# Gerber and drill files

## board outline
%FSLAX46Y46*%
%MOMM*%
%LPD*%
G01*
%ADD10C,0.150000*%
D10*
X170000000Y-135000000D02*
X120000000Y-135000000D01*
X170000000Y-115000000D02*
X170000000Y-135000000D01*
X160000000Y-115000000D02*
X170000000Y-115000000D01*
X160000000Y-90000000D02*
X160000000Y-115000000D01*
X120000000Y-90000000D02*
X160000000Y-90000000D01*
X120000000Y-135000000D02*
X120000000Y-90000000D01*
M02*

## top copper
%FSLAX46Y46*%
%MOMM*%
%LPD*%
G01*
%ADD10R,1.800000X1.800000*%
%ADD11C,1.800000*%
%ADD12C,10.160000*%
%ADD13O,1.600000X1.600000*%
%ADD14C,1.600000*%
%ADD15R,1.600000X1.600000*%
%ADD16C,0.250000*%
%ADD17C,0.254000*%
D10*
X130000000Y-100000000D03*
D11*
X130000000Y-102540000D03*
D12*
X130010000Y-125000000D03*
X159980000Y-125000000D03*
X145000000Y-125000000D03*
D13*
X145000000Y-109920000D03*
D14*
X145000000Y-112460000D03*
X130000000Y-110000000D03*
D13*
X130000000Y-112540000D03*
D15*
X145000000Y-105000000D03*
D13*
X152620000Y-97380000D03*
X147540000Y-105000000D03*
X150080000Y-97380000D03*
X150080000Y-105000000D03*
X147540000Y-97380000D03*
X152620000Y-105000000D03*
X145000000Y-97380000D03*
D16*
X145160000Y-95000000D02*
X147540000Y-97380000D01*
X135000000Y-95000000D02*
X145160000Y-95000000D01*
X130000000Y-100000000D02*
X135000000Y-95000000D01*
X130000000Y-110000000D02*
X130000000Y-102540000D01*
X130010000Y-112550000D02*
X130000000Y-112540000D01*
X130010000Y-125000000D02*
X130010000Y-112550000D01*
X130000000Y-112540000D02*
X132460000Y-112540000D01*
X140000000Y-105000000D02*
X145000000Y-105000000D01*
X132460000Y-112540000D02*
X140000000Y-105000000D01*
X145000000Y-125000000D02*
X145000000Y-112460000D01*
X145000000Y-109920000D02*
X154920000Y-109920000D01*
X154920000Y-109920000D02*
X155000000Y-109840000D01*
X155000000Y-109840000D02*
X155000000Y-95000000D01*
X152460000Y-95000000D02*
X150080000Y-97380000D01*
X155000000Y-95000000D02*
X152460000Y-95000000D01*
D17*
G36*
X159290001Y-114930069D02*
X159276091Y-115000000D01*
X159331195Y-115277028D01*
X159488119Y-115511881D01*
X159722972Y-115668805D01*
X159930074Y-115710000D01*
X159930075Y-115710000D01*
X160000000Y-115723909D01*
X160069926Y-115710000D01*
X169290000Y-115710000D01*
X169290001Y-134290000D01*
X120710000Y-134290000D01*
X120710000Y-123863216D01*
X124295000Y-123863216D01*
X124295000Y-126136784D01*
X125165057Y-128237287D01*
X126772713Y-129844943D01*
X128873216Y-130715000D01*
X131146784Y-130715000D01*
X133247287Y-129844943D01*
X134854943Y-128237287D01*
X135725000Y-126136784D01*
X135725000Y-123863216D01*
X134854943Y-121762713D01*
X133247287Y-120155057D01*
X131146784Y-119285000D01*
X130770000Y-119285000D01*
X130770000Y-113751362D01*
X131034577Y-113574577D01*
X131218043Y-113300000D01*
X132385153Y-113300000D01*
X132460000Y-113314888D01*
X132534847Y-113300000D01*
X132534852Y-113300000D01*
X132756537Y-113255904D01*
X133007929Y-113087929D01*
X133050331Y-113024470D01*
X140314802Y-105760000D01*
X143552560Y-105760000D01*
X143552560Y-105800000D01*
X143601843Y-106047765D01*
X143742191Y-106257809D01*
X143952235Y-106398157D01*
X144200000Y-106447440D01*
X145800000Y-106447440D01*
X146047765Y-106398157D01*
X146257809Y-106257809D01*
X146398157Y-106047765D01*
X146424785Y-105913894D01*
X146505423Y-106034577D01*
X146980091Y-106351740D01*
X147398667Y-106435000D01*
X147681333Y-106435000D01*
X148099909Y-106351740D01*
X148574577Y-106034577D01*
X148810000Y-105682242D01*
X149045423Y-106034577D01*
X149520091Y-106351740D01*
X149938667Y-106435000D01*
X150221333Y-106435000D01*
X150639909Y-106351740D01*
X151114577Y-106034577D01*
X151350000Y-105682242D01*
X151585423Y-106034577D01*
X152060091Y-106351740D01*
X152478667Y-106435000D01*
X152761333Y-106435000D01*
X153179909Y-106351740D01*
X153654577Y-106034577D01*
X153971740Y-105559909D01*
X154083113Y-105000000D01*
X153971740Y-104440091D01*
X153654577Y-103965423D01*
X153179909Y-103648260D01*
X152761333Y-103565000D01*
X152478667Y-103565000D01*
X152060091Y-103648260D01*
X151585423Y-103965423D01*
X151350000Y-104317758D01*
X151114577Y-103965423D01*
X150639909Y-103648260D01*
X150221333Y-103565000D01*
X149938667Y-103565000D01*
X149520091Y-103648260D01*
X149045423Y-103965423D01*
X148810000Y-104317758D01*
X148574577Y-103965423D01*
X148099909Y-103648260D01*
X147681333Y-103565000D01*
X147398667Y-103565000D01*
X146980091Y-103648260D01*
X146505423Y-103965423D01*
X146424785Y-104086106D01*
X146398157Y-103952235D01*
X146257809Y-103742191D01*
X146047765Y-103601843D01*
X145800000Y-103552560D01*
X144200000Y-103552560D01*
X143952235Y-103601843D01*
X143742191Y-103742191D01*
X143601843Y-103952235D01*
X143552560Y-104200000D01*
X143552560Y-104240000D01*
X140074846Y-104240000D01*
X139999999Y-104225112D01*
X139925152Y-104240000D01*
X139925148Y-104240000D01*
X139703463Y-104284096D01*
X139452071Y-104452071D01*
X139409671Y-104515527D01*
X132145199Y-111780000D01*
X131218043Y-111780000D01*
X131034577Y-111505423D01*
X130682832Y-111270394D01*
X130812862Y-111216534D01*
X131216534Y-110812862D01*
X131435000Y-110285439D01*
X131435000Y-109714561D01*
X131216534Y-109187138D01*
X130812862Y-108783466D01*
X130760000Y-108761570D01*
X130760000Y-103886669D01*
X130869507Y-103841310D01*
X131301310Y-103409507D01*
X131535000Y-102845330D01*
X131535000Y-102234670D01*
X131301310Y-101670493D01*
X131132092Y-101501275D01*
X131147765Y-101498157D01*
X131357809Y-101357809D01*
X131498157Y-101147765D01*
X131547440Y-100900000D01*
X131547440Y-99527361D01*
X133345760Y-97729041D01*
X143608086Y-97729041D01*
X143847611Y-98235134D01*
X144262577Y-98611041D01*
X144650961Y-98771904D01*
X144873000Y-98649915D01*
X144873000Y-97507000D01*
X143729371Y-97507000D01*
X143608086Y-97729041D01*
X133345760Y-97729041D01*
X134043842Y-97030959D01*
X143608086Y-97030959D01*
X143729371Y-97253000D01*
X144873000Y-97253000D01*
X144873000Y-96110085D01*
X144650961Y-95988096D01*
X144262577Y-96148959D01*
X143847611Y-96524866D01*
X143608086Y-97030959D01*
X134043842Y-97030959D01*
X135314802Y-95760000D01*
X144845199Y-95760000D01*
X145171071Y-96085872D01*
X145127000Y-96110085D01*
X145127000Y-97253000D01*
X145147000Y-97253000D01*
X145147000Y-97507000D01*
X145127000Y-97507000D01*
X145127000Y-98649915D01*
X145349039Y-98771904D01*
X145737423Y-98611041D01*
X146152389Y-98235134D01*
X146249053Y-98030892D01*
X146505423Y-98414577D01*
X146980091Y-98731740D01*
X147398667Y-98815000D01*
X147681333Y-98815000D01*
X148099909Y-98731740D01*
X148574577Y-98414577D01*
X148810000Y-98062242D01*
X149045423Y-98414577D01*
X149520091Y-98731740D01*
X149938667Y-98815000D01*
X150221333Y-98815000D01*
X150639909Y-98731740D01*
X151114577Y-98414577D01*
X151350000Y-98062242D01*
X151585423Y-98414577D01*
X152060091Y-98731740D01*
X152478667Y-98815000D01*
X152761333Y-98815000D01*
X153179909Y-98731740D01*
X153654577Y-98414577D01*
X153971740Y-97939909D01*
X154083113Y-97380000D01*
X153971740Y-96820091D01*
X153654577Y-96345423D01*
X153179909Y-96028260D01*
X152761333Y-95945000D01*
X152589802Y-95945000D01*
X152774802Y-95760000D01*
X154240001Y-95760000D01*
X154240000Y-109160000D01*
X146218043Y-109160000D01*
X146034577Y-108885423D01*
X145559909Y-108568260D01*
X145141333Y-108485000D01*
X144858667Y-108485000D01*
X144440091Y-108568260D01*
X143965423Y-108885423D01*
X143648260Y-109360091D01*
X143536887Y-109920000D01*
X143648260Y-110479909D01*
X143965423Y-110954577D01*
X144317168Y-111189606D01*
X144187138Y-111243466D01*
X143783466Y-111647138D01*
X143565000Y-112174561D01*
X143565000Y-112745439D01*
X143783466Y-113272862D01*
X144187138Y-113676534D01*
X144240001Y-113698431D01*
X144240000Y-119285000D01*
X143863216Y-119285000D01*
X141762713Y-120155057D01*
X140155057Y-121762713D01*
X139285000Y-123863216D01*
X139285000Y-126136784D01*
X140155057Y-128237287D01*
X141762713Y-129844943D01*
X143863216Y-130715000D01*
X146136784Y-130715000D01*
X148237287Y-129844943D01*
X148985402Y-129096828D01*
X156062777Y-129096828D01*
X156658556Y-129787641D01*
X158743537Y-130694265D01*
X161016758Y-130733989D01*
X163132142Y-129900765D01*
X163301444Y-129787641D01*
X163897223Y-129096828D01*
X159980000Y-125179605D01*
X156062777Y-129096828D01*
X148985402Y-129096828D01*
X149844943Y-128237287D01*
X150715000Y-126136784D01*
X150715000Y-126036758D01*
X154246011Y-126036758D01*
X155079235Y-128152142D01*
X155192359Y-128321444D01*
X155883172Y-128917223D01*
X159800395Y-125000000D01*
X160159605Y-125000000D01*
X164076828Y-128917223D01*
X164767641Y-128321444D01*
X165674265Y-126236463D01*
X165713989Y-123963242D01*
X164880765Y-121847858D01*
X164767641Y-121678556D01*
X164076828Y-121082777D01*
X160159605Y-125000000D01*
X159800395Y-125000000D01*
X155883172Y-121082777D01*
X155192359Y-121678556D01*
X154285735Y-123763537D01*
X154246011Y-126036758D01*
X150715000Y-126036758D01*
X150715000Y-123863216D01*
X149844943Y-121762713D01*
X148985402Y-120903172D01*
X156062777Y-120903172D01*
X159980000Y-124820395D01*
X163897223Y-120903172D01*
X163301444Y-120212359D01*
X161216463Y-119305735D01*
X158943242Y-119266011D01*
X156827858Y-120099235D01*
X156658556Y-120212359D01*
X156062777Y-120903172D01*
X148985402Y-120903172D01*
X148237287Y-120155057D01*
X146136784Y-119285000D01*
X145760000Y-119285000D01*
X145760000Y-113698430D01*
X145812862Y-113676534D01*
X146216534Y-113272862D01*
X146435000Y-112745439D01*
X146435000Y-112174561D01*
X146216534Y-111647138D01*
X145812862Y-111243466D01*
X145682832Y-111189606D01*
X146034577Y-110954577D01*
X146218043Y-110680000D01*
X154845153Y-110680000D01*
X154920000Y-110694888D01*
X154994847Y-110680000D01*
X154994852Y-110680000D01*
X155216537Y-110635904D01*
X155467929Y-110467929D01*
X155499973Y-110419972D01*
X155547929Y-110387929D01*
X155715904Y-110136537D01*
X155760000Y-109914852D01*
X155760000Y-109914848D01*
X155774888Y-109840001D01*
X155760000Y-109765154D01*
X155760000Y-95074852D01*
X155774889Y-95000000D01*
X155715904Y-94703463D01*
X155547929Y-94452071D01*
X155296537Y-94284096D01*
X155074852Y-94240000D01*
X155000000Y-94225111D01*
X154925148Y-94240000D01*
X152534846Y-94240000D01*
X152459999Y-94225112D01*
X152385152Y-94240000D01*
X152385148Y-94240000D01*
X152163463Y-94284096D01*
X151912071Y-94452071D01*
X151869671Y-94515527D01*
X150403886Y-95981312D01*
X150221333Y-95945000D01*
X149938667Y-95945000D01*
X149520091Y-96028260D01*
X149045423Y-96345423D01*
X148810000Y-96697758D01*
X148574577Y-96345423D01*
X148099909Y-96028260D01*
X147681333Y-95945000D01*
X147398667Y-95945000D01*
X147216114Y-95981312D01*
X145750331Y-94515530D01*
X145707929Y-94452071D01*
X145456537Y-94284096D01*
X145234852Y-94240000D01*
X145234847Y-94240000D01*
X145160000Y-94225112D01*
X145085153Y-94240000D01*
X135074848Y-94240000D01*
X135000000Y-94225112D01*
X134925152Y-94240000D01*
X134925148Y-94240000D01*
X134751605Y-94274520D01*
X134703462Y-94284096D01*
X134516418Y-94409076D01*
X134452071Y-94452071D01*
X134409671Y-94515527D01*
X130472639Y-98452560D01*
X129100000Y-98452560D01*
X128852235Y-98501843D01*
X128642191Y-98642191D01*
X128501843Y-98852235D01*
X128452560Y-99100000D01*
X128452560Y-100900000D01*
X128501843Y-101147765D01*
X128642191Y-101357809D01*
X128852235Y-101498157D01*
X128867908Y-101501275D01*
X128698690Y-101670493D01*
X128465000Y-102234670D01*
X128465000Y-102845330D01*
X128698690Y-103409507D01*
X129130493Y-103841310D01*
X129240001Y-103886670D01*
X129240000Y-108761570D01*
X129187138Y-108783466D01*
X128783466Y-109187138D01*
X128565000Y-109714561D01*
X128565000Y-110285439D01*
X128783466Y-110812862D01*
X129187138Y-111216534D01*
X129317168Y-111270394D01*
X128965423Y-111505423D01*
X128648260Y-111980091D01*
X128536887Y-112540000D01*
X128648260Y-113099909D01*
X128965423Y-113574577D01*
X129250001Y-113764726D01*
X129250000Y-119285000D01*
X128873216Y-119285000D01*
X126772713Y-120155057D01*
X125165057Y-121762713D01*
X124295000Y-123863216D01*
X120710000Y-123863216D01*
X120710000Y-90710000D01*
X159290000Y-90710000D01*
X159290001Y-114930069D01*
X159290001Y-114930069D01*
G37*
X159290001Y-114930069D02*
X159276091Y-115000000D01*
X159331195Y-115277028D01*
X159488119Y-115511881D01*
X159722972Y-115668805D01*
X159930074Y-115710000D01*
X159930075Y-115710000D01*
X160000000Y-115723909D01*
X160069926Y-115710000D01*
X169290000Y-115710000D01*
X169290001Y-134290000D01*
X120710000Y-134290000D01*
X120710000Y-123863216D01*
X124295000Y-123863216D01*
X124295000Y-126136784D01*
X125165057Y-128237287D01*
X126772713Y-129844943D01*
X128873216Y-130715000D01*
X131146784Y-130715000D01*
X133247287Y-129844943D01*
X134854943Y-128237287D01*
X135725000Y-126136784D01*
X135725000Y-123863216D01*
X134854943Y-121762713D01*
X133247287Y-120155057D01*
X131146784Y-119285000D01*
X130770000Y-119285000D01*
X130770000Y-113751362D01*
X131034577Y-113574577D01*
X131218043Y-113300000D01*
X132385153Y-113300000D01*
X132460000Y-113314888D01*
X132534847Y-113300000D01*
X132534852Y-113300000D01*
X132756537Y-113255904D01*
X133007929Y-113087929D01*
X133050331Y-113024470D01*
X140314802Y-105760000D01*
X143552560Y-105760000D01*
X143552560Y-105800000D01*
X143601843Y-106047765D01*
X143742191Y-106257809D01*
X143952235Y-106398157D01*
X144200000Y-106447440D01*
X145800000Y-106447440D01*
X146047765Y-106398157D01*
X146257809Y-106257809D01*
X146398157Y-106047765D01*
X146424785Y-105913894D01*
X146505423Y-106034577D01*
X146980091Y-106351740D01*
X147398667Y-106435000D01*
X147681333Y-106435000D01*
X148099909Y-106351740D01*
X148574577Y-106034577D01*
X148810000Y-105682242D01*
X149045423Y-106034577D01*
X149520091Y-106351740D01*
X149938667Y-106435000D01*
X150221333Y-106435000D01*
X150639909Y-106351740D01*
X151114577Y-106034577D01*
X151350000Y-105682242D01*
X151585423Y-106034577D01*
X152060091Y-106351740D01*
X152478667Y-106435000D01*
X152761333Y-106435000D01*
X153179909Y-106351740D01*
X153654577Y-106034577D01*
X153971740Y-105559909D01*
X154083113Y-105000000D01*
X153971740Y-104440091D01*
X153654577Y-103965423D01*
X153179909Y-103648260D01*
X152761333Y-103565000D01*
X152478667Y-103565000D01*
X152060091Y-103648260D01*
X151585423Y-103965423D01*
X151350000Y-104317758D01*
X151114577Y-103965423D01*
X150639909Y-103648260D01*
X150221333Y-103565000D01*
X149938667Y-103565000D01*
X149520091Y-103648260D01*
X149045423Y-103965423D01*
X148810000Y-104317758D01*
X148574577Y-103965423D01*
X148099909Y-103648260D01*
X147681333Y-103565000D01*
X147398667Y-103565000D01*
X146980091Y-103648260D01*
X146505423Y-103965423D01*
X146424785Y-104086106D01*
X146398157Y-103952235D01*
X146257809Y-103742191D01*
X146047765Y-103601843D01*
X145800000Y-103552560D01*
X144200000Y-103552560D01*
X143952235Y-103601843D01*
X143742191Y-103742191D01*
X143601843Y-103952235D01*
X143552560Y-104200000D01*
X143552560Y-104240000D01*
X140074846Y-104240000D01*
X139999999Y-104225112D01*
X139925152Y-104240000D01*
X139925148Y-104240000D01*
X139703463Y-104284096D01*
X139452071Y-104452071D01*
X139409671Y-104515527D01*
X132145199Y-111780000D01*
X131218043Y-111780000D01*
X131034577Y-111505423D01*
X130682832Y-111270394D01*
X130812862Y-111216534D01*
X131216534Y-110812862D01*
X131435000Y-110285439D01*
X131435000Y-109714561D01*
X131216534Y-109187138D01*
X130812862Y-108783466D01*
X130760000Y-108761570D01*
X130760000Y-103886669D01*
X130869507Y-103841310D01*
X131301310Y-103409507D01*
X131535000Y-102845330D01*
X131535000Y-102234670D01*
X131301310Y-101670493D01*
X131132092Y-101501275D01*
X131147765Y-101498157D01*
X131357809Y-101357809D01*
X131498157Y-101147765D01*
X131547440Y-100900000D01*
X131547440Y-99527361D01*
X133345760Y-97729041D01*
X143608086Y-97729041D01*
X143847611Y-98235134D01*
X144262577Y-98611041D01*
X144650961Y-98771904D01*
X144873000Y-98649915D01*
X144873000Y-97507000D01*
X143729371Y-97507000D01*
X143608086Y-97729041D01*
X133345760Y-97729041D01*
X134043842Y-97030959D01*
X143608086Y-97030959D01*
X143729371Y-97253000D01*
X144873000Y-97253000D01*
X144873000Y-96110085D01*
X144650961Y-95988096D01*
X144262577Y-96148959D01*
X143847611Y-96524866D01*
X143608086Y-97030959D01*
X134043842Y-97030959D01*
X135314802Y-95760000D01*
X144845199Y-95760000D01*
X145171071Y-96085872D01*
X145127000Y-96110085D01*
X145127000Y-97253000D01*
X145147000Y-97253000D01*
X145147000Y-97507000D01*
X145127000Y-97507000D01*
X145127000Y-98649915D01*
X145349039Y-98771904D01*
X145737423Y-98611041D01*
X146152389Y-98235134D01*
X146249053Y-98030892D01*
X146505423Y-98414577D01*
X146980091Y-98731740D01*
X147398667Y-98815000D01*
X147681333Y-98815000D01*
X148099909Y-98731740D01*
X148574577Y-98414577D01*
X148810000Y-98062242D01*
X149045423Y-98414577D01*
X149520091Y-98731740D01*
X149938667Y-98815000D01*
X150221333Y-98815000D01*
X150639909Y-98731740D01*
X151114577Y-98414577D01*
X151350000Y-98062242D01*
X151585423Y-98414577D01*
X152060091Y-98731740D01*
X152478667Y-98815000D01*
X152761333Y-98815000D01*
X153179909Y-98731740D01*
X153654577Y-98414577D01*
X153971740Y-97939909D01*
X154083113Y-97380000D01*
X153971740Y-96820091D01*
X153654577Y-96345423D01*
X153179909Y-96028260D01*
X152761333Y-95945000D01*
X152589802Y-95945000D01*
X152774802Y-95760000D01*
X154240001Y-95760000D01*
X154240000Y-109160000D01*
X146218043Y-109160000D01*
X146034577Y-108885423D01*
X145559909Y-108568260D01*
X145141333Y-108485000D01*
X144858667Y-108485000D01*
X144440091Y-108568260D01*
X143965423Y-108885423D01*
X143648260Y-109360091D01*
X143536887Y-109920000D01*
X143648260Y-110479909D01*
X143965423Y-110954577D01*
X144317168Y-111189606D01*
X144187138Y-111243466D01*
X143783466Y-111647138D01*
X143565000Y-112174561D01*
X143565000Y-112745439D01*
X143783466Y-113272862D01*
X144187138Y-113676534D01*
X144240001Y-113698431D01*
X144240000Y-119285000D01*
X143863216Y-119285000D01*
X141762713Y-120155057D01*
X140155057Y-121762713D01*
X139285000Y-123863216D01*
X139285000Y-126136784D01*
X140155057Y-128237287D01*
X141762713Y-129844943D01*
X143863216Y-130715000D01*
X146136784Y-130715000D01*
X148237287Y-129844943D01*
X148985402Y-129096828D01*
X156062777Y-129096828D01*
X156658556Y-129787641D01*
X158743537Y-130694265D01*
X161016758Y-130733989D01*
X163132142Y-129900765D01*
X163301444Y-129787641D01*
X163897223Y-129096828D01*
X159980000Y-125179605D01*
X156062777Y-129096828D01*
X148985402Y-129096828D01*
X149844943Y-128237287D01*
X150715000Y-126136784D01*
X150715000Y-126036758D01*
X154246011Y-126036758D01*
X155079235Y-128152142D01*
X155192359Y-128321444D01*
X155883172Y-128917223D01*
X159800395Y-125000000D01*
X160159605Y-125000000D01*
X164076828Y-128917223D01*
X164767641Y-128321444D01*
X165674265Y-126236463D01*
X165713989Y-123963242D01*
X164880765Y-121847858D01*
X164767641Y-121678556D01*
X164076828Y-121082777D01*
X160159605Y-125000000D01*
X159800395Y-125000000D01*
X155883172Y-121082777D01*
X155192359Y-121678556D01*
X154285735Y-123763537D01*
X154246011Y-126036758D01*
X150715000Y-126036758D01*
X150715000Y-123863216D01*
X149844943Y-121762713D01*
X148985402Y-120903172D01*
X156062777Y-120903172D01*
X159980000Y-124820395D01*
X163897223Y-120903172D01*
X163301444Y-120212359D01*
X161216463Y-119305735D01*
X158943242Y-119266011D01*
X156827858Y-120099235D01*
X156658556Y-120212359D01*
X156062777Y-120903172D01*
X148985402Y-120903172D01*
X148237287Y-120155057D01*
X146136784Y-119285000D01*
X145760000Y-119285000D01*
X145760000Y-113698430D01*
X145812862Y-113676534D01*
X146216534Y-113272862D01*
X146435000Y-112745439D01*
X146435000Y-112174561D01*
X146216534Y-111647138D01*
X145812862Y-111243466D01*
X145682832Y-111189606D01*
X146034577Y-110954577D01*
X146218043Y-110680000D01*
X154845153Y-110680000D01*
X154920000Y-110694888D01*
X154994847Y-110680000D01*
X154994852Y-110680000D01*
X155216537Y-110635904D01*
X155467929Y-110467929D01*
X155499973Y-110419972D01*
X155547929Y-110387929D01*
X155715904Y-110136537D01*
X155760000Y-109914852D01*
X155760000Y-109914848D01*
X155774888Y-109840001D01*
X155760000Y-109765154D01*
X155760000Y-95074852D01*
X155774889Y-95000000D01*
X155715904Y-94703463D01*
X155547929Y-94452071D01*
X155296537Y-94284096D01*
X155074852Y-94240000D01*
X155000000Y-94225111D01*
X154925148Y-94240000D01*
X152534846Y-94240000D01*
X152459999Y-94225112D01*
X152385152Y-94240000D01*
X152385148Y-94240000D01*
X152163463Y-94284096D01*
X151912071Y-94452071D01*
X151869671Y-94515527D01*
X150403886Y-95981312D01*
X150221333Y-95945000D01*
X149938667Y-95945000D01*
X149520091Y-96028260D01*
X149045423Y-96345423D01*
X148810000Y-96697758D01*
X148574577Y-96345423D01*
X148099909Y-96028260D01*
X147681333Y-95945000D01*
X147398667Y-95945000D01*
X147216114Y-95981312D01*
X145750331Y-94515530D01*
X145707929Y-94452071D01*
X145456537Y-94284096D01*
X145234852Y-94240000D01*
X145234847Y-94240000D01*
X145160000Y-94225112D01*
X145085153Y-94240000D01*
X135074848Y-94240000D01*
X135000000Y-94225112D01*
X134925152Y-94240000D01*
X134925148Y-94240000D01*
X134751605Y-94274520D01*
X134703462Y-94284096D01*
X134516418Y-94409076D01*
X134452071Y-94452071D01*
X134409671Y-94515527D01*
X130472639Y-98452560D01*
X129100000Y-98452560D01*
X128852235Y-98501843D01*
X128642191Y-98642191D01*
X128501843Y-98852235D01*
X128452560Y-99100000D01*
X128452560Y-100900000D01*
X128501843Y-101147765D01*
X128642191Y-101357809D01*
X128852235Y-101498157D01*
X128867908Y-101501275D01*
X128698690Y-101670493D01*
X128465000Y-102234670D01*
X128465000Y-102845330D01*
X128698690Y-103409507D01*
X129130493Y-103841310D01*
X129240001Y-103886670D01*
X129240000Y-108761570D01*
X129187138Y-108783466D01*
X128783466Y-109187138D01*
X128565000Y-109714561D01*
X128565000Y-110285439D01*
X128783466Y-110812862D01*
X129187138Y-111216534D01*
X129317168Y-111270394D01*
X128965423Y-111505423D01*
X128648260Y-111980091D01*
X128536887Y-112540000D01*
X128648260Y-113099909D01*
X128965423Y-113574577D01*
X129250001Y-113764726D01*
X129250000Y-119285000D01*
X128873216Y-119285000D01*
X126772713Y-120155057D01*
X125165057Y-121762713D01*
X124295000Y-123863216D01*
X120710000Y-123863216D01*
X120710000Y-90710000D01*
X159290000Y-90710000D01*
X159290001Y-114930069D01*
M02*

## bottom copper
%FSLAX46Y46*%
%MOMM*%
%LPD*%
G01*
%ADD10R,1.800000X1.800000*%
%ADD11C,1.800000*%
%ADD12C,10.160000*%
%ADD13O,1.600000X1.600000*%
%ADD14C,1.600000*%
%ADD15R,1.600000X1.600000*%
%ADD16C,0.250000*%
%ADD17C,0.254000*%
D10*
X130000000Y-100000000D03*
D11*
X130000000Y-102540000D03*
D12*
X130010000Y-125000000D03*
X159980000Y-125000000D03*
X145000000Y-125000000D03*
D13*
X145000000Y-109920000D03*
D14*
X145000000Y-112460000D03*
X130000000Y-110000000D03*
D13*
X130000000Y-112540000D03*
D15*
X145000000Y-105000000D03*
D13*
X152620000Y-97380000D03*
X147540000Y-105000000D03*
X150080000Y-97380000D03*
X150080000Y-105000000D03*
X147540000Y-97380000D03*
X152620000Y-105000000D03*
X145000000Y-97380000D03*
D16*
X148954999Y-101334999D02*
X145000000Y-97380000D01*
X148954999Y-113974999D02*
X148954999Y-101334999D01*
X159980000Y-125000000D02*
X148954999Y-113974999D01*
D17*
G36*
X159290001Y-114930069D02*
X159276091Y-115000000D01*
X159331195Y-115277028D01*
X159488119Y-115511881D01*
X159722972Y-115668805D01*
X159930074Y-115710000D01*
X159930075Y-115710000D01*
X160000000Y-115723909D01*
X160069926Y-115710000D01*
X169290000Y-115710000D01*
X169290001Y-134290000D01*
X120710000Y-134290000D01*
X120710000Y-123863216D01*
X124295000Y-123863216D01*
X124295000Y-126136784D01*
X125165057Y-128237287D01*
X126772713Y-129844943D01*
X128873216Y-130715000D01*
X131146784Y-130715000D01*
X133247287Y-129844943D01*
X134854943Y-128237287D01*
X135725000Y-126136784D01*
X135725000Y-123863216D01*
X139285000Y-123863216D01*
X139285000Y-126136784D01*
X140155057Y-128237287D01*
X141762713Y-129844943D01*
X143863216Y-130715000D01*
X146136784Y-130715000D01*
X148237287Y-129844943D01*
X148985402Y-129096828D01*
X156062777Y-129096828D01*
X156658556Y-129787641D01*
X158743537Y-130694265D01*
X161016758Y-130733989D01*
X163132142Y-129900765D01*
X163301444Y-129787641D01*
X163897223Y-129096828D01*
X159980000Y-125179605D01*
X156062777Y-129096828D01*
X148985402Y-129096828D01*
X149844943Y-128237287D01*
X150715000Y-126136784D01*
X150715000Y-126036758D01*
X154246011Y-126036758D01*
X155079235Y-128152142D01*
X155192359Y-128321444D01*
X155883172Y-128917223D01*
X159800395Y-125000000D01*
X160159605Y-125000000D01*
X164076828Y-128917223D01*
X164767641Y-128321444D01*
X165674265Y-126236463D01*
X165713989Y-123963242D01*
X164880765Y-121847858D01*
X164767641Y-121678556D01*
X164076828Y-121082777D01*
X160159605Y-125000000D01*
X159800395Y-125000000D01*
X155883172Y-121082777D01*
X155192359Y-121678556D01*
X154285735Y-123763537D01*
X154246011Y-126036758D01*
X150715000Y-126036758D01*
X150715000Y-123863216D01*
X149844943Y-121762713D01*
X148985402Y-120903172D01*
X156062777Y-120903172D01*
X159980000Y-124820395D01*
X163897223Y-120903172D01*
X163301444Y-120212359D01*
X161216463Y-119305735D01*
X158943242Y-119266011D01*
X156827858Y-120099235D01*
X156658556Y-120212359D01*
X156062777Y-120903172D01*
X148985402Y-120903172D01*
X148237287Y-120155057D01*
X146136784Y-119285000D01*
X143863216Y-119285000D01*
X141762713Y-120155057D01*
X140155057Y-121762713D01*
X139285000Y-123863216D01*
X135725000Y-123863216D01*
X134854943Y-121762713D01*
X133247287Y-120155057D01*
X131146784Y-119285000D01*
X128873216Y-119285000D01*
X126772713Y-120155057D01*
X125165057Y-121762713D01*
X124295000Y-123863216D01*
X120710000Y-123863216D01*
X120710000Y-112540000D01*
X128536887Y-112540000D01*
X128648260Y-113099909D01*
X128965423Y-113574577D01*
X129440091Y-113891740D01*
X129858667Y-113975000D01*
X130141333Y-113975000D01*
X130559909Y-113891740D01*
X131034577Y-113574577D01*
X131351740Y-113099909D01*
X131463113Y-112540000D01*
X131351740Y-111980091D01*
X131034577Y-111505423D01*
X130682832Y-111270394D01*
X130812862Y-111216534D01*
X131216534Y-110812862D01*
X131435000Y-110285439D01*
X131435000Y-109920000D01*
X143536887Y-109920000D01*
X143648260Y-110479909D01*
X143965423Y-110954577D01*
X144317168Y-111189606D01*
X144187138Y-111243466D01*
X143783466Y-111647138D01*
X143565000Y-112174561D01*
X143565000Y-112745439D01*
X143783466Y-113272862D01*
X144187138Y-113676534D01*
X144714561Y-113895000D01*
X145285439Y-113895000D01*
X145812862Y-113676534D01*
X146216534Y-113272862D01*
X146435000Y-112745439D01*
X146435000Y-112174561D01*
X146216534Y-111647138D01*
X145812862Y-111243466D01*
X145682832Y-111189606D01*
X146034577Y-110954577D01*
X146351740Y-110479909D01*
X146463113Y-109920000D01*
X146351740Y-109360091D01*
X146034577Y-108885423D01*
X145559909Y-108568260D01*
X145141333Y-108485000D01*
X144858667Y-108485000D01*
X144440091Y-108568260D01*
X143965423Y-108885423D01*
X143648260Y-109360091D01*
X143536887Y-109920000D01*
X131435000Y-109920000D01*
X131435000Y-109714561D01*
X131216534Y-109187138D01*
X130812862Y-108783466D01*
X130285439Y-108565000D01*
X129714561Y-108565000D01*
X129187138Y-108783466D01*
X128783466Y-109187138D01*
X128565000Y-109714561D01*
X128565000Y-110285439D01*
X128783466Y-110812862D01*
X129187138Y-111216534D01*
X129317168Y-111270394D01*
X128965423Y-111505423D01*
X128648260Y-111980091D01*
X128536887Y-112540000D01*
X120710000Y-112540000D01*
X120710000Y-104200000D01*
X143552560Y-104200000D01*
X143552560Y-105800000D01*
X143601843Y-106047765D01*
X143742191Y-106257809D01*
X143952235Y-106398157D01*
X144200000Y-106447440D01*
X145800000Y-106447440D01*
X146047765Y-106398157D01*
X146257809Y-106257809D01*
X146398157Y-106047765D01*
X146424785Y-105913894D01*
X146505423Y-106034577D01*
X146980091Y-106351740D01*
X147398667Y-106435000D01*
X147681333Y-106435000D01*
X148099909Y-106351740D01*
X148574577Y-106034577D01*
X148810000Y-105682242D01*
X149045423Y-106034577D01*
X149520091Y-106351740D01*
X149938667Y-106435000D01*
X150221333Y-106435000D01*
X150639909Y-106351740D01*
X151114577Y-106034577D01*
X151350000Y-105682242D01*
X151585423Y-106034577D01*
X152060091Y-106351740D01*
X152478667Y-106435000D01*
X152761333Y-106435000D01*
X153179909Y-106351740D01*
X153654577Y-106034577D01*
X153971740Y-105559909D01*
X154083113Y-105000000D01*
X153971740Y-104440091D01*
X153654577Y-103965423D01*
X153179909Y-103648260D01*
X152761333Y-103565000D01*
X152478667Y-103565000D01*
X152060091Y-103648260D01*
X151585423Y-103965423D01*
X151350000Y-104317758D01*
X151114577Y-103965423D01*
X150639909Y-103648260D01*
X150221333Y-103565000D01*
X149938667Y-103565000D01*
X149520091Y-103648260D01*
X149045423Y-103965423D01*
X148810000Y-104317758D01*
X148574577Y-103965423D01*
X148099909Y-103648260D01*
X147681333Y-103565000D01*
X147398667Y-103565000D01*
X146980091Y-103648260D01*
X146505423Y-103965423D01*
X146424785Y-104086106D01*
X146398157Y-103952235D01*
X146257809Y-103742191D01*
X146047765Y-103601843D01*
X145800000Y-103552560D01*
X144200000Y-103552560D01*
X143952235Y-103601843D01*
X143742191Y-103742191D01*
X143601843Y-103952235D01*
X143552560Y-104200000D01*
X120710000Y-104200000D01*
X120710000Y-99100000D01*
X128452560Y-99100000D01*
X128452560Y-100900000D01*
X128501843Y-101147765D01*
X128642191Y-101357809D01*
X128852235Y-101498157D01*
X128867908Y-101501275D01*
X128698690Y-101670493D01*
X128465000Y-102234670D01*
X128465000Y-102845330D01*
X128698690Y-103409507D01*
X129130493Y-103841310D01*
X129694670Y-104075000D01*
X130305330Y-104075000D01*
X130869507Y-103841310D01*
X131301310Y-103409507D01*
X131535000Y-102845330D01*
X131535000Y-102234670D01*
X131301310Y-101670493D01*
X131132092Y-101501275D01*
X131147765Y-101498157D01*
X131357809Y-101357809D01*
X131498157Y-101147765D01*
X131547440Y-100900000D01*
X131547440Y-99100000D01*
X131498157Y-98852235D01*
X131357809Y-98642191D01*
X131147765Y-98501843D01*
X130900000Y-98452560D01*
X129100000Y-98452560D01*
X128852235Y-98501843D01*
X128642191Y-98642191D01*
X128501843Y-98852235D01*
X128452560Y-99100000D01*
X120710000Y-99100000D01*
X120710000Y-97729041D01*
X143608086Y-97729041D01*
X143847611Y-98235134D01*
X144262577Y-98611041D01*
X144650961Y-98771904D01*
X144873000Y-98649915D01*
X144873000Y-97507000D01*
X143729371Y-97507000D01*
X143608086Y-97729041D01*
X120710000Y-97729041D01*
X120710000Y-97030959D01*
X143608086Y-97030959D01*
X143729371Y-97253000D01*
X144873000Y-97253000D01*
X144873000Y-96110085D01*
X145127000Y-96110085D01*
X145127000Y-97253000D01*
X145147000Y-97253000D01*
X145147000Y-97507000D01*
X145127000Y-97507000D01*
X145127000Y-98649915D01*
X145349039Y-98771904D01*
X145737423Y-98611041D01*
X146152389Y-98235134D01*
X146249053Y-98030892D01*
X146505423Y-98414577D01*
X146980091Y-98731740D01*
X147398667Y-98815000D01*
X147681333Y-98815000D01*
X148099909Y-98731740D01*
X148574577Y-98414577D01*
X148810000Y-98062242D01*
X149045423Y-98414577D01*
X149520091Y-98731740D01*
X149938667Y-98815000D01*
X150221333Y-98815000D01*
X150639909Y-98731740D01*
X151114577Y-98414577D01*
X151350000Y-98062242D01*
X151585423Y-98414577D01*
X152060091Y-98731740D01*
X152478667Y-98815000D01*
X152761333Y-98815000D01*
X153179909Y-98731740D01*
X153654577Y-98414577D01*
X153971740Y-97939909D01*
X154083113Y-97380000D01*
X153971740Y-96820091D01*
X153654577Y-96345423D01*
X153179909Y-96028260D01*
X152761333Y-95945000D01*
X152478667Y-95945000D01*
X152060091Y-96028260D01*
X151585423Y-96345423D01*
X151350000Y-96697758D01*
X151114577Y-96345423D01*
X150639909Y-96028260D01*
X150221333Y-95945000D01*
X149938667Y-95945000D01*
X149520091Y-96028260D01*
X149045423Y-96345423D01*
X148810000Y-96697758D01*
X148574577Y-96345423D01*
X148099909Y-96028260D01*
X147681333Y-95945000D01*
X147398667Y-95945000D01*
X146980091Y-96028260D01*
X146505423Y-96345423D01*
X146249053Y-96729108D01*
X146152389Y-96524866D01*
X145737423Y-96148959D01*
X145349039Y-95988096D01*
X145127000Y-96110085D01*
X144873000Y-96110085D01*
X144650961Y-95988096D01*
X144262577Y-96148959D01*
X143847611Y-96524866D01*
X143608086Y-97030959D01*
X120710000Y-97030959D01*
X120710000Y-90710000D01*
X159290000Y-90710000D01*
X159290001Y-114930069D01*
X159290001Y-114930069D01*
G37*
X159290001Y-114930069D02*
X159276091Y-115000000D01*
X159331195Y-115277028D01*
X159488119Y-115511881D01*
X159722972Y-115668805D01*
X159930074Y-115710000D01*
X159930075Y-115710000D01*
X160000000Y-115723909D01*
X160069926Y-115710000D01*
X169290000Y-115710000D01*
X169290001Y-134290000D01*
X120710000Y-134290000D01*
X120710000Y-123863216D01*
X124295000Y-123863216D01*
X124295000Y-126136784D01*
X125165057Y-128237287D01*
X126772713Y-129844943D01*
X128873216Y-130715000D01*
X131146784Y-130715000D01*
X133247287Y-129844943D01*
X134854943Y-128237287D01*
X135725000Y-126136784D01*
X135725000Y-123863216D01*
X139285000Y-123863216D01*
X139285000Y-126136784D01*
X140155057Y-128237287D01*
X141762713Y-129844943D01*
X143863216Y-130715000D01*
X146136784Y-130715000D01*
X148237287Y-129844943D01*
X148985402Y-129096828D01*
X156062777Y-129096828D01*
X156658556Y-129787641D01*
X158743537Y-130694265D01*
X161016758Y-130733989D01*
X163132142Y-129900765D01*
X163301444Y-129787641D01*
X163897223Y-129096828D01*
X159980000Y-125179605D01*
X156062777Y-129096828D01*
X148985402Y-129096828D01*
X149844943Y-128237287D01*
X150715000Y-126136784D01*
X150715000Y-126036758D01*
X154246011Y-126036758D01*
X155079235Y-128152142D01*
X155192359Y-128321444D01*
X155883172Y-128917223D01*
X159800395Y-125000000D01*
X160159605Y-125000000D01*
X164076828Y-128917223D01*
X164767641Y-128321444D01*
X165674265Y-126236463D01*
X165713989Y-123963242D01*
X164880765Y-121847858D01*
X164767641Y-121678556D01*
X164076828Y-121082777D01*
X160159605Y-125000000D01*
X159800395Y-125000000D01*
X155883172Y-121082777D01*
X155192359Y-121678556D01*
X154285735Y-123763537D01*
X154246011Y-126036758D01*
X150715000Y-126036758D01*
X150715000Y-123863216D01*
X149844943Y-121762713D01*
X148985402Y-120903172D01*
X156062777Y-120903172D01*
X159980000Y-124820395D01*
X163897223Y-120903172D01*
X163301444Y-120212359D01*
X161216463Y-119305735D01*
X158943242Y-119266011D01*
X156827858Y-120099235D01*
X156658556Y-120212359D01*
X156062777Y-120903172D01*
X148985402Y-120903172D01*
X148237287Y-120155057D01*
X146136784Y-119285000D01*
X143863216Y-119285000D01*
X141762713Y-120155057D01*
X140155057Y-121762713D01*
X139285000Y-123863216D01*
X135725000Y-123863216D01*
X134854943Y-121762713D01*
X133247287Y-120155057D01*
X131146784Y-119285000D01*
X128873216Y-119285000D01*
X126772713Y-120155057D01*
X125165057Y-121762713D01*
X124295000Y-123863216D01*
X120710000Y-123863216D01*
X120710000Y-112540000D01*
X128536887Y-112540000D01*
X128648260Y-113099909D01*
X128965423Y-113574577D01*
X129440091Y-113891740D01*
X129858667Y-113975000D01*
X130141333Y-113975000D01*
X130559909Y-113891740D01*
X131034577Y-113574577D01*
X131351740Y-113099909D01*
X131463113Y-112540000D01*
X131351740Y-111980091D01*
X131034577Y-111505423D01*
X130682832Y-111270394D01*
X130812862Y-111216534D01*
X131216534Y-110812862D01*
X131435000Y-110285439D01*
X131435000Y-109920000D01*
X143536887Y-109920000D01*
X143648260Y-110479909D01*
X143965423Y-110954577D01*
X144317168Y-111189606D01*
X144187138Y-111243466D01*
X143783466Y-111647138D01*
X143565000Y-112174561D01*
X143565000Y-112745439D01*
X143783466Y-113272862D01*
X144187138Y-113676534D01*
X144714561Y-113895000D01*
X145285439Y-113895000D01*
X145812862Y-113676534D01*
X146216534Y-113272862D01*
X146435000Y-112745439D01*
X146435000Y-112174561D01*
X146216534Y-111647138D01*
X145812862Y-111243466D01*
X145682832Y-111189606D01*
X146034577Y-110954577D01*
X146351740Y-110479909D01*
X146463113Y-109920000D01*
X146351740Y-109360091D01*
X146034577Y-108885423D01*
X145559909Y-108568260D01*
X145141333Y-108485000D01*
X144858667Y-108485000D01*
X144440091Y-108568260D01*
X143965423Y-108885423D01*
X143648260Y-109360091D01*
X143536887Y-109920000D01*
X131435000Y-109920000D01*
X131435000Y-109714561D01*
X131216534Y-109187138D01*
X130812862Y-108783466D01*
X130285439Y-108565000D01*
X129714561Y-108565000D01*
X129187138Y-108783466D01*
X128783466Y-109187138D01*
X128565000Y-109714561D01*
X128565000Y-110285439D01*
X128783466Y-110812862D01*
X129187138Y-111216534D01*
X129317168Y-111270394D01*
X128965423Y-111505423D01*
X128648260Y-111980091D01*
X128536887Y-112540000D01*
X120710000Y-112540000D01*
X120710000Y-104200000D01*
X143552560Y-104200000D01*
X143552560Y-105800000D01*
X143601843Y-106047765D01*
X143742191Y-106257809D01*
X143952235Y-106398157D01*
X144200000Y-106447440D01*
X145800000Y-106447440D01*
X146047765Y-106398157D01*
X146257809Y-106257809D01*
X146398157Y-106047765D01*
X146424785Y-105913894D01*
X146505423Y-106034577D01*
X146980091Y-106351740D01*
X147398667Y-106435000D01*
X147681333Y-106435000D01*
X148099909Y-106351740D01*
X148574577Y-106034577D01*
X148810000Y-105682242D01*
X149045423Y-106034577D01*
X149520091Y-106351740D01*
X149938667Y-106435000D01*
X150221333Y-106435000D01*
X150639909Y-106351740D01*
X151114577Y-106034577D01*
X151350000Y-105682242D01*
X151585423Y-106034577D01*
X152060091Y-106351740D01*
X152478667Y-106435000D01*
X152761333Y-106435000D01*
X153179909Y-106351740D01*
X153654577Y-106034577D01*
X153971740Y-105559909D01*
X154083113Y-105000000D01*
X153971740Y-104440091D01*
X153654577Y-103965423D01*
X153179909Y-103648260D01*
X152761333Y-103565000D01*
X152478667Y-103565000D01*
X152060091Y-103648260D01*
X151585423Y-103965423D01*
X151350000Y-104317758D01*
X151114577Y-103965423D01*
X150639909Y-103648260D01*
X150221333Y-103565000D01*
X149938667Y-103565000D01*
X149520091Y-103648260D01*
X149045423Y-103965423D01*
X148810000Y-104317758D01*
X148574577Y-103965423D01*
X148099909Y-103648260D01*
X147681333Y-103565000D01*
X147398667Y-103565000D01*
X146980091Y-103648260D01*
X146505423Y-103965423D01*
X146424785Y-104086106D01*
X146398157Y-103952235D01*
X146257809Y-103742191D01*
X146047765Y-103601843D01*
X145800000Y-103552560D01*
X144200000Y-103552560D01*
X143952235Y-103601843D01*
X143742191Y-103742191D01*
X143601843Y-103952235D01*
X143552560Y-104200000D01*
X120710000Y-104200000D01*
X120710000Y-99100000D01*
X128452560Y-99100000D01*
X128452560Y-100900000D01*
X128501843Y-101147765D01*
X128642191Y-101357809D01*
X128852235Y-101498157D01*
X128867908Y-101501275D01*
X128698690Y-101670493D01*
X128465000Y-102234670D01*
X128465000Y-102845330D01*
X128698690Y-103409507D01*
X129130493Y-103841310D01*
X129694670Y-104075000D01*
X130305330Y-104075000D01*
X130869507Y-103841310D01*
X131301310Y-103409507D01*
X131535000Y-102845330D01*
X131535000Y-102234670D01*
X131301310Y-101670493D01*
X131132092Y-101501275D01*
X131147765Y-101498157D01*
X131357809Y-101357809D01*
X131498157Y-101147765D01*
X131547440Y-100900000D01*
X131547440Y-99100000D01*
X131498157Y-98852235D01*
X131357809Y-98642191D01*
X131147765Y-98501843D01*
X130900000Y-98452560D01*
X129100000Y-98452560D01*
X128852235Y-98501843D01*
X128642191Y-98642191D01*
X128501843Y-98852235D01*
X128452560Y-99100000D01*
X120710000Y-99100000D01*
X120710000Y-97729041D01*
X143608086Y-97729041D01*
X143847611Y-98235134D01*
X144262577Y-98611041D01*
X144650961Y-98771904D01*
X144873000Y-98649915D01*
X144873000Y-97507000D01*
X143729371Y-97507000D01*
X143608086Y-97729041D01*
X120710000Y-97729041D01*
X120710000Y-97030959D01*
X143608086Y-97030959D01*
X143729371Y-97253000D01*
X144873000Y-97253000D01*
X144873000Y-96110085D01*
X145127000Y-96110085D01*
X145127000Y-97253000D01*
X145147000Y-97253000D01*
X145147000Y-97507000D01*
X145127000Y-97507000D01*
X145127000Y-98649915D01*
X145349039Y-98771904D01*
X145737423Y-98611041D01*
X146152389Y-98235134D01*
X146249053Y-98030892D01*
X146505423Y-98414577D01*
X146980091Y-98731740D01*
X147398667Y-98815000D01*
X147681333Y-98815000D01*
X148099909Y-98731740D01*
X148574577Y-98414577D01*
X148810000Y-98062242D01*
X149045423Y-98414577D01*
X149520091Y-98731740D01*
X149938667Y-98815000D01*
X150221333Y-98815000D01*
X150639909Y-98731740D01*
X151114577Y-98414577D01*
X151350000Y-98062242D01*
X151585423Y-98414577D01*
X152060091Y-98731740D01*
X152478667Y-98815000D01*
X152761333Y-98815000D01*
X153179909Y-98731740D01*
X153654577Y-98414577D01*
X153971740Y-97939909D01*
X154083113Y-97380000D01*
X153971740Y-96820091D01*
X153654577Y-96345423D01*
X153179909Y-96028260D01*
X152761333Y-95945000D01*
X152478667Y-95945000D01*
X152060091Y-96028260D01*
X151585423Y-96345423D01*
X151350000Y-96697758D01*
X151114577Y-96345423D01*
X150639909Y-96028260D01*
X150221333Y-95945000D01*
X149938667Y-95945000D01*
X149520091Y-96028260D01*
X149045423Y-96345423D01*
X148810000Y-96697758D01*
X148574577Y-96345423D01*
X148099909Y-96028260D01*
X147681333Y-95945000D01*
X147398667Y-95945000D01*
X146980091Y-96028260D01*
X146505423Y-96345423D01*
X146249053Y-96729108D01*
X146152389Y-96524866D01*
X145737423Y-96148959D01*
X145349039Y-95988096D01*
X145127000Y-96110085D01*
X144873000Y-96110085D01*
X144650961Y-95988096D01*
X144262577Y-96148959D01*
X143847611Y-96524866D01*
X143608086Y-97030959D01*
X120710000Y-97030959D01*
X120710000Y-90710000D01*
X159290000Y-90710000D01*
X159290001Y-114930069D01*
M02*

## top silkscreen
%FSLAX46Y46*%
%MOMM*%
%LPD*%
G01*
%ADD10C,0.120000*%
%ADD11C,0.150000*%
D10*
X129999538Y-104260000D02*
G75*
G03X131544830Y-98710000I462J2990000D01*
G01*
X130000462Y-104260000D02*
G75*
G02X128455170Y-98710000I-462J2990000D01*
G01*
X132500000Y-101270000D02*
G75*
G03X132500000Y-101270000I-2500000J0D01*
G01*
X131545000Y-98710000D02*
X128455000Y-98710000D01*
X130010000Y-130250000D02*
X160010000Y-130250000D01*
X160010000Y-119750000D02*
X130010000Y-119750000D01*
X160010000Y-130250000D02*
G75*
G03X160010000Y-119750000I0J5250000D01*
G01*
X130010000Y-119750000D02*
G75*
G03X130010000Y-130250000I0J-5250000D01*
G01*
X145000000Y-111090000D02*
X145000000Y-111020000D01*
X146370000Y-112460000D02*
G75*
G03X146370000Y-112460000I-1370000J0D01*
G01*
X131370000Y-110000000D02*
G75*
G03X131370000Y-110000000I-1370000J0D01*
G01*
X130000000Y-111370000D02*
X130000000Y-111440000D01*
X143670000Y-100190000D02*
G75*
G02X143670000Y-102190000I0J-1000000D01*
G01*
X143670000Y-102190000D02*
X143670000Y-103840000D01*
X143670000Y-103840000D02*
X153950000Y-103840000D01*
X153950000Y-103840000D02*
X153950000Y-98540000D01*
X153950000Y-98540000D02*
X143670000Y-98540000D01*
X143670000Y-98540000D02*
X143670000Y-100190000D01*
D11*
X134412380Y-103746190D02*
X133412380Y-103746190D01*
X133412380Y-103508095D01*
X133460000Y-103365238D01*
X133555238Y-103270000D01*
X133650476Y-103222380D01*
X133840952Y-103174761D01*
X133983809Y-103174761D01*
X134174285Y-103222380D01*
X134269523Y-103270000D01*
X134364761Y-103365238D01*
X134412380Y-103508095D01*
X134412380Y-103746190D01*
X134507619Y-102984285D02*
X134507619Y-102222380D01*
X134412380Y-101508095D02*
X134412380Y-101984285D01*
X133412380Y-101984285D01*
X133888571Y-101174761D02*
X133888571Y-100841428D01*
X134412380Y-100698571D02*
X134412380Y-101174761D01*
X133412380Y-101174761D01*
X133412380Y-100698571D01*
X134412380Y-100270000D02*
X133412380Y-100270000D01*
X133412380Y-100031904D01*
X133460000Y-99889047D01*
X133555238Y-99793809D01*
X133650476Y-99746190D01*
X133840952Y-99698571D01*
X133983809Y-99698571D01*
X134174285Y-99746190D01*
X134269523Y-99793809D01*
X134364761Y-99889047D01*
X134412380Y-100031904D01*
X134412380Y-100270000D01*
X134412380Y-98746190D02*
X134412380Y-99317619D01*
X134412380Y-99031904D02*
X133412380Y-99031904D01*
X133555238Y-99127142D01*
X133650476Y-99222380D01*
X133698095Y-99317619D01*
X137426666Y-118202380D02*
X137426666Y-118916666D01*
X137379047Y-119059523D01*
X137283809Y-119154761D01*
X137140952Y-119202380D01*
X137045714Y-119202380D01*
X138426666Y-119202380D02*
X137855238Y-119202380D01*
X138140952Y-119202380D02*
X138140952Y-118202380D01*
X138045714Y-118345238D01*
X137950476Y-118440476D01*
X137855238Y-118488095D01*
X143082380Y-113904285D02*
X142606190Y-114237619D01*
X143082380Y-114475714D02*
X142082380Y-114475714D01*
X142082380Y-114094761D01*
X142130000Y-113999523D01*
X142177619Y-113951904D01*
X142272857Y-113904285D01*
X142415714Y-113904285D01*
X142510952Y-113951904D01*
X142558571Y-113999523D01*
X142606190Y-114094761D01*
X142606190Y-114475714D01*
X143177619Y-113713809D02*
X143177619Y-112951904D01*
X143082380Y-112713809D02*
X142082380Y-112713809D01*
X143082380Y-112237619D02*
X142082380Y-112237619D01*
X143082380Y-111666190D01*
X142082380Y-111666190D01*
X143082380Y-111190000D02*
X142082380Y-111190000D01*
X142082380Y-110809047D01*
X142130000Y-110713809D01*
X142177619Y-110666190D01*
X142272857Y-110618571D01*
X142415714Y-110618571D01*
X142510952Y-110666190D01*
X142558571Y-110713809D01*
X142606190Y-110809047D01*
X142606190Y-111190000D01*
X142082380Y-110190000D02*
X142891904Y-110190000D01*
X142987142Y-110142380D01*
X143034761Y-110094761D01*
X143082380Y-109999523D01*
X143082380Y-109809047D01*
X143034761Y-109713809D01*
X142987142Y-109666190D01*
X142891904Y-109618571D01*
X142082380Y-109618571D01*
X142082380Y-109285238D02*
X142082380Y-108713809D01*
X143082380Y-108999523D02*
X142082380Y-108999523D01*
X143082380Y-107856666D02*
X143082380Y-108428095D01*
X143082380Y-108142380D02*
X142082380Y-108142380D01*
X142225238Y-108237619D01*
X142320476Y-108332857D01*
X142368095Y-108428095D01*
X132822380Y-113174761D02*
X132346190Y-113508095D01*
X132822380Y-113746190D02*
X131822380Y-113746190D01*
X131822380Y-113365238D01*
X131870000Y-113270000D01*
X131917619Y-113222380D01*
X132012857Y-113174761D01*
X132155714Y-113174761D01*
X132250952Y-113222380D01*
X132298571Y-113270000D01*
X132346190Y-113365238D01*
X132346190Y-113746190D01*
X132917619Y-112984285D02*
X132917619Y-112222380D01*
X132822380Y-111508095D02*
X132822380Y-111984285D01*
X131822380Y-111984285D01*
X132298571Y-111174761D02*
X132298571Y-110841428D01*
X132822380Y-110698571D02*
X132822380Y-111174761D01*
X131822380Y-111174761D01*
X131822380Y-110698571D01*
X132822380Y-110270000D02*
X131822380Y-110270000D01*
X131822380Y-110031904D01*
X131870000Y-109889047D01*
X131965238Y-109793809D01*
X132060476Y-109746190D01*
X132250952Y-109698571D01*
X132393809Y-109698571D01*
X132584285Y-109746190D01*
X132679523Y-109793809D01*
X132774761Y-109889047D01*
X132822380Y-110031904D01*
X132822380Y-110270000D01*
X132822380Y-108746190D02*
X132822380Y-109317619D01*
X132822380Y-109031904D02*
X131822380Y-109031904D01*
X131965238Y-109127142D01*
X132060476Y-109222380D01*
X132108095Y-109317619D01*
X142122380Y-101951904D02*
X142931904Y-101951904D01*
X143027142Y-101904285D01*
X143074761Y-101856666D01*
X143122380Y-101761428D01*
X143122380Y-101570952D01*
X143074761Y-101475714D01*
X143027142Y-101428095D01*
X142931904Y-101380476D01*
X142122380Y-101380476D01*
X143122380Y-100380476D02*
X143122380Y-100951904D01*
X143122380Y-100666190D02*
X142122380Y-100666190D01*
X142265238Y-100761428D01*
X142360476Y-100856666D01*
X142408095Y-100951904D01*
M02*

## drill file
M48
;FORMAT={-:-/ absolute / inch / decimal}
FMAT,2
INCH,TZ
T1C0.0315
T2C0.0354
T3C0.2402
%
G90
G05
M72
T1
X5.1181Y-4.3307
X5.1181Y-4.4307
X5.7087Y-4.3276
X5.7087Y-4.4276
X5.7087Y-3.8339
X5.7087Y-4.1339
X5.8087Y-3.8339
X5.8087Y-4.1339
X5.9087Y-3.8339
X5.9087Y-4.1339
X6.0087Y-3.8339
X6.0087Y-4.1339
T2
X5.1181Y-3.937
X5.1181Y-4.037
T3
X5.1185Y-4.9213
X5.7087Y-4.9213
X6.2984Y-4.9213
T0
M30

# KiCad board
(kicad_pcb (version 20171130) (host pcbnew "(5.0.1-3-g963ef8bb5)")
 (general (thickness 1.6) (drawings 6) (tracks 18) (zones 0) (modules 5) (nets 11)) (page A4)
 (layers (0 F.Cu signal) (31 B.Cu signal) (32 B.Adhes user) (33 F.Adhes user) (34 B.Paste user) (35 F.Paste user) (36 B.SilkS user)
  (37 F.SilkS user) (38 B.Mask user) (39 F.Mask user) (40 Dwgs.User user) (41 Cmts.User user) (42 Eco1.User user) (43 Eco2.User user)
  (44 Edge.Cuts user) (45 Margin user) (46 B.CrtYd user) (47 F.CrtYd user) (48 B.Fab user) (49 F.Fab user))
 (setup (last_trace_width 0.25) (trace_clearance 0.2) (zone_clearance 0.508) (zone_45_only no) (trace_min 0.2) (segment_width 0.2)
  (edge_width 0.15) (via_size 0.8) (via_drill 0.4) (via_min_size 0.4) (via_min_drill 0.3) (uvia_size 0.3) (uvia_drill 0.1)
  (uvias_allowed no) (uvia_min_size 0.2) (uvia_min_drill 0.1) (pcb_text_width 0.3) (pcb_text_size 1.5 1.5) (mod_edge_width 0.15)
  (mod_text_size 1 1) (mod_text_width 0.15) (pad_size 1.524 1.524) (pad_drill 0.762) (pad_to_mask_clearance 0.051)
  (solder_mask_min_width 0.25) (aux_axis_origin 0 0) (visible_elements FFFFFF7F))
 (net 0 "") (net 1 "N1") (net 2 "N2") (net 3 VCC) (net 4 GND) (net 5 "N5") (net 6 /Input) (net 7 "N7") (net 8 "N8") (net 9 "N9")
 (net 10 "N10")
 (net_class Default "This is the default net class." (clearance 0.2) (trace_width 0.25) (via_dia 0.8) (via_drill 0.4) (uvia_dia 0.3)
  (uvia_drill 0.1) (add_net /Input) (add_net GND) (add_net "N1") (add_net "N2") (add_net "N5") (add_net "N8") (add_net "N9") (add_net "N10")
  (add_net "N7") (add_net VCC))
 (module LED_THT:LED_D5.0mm (layer F.Cu) (at 130 100 270)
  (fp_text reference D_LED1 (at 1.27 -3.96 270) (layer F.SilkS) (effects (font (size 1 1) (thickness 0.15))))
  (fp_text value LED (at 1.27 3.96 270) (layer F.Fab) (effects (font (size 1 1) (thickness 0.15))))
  (fp_arc (start 1.27 0) (end -1.29 -1.54483) (angle 148.9) (layer F.SilkS) (width 0.12))
  (fp_arc (start 1.27 0) (end -1.29 1.54483) (angle -148.9) (layer F.SilkS) (width 0.12))
  (fp_circle (center 1.27 0) (end 3.77 0) (layer F.SilkS) (width 0.12))
  (fp_line (start -1.29 -1.545) (end -1.29 1.545) (layer F.SilkS) (width 0.12))
  (pad 1 thru_hole rect (at 0 0 270) (size 1.8 1.8) (drill 0.9) (layers *.Cu *.Mask) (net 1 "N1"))
  (pad 2 thru_hole circle (at 2.54 0 270) (size 1.8 1.8) (drill 0.9) (layers *.Cu *.Mask) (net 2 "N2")))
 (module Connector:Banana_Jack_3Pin (layer F.Cu) (at 130.01 125)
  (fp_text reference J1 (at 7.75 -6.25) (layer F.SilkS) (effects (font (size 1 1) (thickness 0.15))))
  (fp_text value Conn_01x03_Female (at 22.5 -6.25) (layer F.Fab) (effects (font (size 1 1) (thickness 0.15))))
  (fp_line (start 0 5.25) (end 30 5.25) (layer F.SilkS) (width 0.12))
  (fp_line (start 30 -5.25) (end 0 -5.25) (layer F.SilkS) (width 0.12))
  (fp_arc (start 30 0) (end 30 -5.25) (angle 180) (layer F.SilkS) (width 0.12))
  (fp_arc (start 0 0) (end 0 5.25) (angle 180) (layer F.SilkS) (width 0.12))
  (pad 1 thru_hole circle (at 0 0) (size 10.16 10.16) (drill 6.1) (layers *.Cu *.Mask) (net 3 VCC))
  (pad 3 thru_hole circle (at 29.97 0) (size 10.16 10.16) (drill 6.1) (layers *.Cu *.Mask) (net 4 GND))
  (pad 2 thru_hole circle (at 14.99 0) (size 10.16 10.16) (drill 6.1) (layers *.Cu *.Mask) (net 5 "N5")))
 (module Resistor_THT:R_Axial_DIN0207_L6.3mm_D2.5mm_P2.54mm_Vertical (layer F.Cu) (at 145 112.46 90)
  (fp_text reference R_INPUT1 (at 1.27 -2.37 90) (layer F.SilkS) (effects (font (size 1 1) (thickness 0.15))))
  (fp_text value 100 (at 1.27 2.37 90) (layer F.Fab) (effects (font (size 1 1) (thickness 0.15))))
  (fp_line (start 1.37 0) (end 1.44 0) (layer F.SilkS) (width 0.12))
  (fp_circle (center 0 0) (end 1.37 0) (layer F.SilkS) (width 0.12))
  (pad 2 thru_hole oval (at 2.54 0 90) (size 1.6 1.6) (drill 0.8) (layers *.Cu *.Mask) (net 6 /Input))
  (pad 1 thru_hole circle (at 0 0 90) (size 1.6 1.6) (drill 0.8) (layers *.Cu *.Mask) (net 5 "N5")))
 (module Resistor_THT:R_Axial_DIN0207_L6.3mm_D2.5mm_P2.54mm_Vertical (layer F.Cu) (at 130 110 270)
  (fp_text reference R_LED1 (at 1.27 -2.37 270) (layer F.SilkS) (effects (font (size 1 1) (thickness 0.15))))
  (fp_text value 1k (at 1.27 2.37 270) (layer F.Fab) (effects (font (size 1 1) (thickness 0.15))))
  (fp_circle (center 0 0) (end 1.37 0) (layer F.SilkS) (width 0.12))
  (fp_line (start 1.37 0) (end 1.44 0) (layer F.SilkS) (width 0.12))
  (pad 1 thru_hole circle (at 0 0 270) (size 1.6 1.6) (drill 0.8) (layers *.Cu *.Mask) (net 2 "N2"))
  (pad 2 thru_hole oval (at 2.54 0 270) (size 1.6 1.6) (drill 0.8) (layers *.Cu *.Mask) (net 3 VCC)))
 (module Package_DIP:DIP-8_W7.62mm (layer F.Cu) (at 145 105 90)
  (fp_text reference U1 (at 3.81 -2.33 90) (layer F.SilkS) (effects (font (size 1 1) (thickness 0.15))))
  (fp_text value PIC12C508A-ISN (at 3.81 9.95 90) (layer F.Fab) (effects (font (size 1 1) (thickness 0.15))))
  (fp_arc (start 3.81 -1.33) (end 2.81 -1.33) (angle -180) (layer F.SilkS) (width 0.12))
  (fp_line (start 2.81 -1.33) (end 1.16 -1.33) (layer F.SilkS) (width 0.12))
  (fp_line (start 1.16 -1.33) (end 1.16 8.95) (layer F.SilkS) (width 0.12))
  (fp_line (start 1.16 8.95) (end 6.46 8.95) (layer F.SilkS) (width 0.12))
  (fp_line (start 6.46 8.95) (end 6.46 -1.33) (layer F.SilkS) (width 0.12))
  (fp_line (start 6.46 -1.33) (end 4.81 -1.33) (layer F.SilkS) (width 0.12))
  (pad 1 thru_hole rect (at 0 0 90) (size 1.6 1.6) (drill 0.8) (layers *.Cu *.Mask) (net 3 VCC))
  (pad 5 thru_hole oval (at 7.62 7.62 90) (size 1.6 1.6) (drill 0.8) (layers *.Cu *.Mask) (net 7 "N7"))
  (pad 2 thru_hole oval (at 0 2.54 90) (size 1.6 1.6) (drill 0.8) (layers *.Cu *.Mask) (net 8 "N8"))
  (pad 6 thru_hole oval (at 7.62 5.08 90) (size 1.6 1.6) (drill 0.8) (layers *.Cu *.Mask) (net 6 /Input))
  (pad 3 thru_hole oval (at 0 5.08 90) (size 1.6 1.6) (drill 0.8) (layers *.Cu *.Mask) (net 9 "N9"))
  (pad 7 thru_hole oval (at 7.62 2.54 90) (size 1.6 1.6) (drill 0.8) (layers *.Cu *.Mask) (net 1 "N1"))
  (pad 4 thru_hole oval (at 0 7.62 90) (size 1.6 1.6) (drill 0.8) (layers *.Cu *.Mask) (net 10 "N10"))
  (pad 8 thru_hole oval (at 7.62 0 90) (size 1.6 1.6) (drill 0.8) (layers *.Cu *.Mask) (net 4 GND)))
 (gr_line (start 170 135) (end 120 135) (layer Edge.Cuts) (width 0.15))
 (gr_line (start 170 115) (end 170 135) (layer Edge.Cuts) (width 0.15))
 (gr_line (start 160 115) (end 170 115) (layer Edge.Cuts) (width 0.15))
 (gr_line (start 160 90) (end 160 115) (layer Edge.Cuts) (width 0.15))
 (gr_line (start 120 90) (end 160 90) (layer Edge.Cuts) (width 0.15))
 (gr_line (start 120 135) (end 120 90) (layer Edge.Cuts) (width 0.15))
 (segment (start 145.16 95) (end 147.54 97.38) (width 0.25) (layer F.Cu) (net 1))
 (segment (start 135 95) (end 145.16 95) (width 0.25) (layer F.Cu) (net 1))
 (segment (start 130 100) (end 135 95) (width 0.25) (layer F.Cu) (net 1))
 (segment (start 130 110) (end 130 102.54) (width 0.25) (layer F.Cu) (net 2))
 (segment (start 130.01 112.55) (end 130 112.54) (width 0.25) (layer F.Cu) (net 3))
 (segment (start 130.01 125) (end 130.01 112.55) (width 0.25) (layer F.Cu) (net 3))
 (segment (start 130 112.54) (end 132.46 112.54) (width 0.25) (layer F.Cu) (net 3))
 (segment (start 140 105) (end 145 105) (width 0.25) (layer F.Cu) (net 3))
 (segment (start 132.46 112.54) (end 140 105) (width 0.25) (layer F.Cu) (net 3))
 (segment (start 148.954999 101.334999) (end 145 97.38) (width 0.25) (layer B.Cu) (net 4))
 (segment (start 148.954999 113.974999) (end 148.954999 101.334999) (width 0.25) (layer B.Cu) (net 4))
 (segment (start 159.98 125) (end 148.954999 113.974999) (width 0.25) (layer B.Cu) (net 4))
 (segment (start 145 125) (end 145 112.46) (width 0.25) (layer F.Cu) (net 5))
 (segment (start 145 109.92) (end 154.92 109.92) (width 0.25) (layer F.Cu) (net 6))
 (segment (start 154.92 109.92) (end 155 109.84) (width 0.25) (layer F.Cu) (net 6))
 (segment (start 155 109.84) (end 155 95) (width 0.25) (layer F.Cu) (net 6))
 (segment (start 152.46 95) (end 150.08 97.38) (width 0.25) (layer F.Cu) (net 6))
 (segment (start 155 95) (end 152.46 95) (width 0.25) (layer F.Cu) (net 6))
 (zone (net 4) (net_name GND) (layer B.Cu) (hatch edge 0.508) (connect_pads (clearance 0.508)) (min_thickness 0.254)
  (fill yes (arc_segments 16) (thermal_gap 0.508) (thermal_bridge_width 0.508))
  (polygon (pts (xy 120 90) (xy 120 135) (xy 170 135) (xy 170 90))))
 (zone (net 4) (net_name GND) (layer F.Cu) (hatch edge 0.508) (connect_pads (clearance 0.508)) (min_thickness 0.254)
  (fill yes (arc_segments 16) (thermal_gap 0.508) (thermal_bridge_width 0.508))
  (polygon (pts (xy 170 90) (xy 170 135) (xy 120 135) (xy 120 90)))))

